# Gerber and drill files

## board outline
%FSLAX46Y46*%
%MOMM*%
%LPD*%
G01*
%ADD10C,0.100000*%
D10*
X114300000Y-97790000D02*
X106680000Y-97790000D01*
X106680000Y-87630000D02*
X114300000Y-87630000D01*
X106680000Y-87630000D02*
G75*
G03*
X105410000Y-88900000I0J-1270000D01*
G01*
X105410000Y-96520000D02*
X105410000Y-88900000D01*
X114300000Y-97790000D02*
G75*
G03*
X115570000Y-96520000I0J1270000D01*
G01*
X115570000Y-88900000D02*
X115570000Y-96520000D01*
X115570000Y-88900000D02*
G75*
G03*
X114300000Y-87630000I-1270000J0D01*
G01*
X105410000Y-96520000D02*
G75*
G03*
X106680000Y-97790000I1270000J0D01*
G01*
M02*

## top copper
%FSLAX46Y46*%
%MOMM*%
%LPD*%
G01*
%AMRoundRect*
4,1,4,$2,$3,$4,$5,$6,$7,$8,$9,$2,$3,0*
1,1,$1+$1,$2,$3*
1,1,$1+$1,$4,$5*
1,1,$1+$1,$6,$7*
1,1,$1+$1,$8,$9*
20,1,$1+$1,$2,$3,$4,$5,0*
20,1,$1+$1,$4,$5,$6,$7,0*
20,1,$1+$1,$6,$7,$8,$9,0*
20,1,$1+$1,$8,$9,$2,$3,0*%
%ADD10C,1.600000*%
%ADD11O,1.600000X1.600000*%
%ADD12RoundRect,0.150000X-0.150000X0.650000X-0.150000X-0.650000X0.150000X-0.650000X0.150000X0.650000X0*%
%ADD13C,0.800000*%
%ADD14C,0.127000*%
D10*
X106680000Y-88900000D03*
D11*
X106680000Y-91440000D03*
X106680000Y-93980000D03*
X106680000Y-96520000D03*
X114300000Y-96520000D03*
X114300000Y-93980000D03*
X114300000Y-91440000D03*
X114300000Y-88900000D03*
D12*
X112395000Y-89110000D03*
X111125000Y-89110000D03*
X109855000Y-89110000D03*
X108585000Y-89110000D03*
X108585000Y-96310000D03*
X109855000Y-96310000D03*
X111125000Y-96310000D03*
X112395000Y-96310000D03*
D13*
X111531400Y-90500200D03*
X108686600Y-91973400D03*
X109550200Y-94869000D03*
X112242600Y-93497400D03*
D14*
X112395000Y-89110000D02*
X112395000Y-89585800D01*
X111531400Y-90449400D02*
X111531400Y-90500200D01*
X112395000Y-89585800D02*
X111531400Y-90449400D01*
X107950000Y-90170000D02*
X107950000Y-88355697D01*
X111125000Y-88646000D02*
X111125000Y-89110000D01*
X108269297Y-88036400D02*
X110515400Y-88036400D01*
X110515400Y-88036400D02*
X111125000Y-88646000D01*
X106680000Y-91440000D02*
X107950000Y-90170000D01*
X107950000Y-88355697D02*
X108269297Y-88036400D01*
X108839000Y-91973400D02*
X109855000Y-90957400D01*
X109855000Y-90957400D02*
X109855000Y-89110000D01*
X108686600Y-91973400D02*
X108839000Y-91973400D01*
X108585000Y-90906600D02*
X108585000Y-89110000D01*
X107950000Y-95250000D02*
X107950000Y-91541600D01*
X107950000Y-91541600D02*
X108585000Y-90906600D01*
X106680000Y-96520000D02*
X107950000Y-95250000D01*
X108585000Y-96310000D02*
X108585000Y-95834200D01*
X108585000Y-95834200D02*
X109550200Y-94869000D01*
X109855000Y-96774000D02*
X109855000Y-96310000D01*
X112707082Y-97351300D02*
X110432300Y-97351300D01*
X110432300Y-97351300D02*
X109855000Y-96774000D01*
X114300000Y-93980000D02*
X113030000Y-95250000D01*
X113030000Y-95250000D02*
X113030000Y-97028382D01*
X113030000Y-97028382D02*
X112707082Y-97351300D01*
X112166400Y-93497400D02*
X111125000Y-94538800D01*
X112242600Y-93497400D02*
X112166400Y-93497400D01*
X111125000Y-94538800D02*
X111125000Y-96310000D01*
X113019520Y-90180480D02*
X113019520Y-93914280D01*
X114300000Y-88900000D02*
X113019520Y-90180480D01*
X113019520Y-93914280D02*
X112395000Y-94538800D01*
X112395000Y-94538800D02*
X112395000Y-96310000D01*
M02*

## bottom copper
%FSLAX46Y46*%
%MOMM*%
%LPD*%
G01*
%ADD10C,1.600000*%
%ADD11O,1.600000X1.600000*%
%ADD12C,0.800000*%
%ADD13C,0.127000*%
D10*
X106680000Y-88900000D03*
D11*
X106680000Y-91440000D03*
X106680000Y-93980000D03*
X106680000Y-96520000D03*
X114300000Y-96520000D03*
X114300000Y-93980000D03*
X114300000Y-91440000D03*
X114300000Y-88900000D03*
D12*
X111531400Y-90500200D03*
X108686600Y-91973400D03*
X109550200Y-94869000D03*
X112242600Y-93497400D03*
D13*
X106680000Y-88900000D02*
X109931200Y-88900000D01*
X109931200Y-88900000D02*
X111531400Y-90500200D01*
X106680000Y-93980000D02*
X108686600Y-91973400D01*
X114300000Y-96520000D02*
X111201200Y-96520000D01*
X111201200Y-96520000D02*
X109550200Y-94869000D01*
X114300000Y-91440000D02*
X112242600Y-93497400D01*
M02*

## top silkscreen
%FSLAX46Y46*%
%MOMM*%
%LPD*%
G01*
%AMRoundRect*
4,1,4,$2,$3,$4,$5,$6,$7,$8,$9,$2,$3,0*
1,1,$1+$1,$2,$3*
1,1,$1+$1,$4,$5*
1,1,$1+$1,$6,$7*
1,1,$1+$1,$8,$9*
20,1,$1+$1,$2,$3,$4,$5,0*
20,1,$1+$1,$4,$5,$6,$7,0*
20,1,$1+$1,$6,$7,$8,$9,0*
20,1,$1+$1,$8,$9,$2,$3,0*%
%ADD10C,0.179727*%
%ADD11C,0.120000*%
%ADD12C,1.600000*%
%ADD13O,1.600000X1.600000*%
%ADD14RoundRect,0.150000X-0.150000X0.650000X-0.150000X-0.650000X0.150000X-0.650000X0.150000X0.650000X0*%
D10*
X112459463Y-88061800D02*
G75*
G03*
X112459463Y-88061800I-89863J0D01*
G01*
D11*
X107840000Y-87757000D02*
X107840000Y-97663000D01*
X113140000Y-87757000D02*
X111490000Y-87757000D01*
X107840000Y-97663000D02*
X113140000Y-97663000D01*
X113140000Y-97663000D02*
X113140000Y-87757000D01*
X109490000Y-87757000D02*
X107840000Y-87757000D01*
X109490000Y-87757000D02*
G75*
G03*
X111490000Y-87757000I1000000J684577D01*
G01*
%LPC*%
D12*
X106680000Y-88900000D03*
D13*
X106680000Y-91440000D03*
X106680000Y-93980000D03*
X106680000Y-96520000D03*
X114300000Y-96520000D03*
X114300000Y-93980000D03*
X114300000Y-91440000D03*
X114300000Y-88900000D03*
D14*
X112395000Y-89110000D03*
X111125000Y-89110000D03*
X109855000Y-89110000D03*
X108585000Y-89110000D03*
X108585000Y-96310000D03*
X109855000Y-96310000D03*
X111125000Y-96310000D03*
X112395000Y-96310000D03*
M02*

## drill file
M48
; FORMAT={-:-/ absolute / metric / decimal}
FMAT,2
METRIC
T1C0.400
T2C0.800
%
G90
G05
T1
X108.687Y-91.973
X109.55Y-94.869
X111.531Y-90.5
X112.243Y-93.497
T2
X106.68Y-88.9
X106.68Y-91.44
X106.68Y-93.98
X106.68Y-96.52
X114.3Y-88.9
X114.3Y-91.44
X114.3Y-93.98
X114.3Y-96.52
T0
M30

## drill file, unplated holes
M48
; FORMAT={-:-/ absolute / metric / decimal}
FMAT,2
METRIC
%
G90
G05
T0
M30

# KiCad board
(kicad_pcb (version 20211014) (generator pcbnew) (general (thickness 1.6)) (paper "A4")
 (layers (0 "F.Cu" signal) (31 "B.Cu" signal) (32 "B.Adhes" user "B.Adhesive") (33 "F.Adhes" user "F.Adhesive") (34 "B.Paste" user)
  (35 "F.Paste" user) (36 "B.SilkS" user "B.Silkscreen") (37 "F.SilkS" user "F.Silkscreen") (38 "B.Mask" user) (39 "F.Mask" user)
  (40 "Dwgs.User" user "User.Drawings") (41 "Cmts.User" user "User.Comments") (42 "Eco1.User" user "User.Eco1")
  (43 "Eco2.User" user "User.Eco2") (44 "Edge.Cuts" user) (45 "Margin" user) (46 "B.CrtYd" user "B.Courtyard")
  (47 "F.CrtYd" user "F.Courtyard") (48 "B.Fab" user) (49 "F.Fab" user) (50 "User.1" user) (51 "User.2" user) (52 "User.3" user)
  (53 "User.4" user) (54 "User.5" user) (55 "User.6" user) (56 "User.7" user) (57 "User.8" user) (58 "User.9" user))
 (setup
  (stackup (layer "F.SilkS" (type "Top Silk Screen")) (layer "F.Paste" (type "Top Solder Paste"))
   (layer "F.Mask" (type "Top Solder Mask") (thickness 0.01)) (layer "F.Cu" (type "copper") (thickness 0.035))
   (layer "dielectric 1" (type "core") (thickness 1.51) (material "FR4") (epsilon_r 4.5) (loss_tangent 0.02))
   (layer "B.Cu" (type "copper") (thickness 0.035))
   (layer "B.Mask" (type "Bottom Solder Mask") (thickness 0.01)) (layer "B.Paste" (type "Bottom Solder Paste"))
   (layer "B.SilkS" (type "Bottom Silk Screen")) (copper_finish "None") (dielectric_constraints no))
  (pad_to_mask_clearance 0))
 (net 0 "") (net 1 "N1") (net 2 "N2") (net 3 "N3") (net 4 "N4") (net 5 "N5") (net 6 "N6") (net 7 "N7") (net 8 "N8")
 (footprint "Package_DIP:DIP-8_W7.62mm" (layer "F.Cu") (at 106.68 88.9)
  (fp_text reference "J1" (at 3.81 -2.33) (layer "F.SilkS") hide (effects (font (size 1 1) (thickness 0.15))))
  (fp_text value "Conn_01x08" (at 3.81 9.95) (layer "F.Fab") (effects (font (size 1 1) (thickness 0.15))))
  (fp_line (start 1.16 -1.143) (end 1.16 8.763) (layer "F.SilkS") (width 0.12))
  (fp_line (start 6.46 -1.143) (end 4.81 -1.143) (layer "F.SilkS") (width 0.12))
  (fp_line (start 1.16 8.763) (end 6.46 8.763) (layer "F.SilkS") (width 0.12))
  (fp_line (start 6.46 8.763) (end 6.46 -1.143) (layer "F.SilkS") (width 0.12))
  (fp_line (start 2.81 -1.143) (end 1.16 -1.143) (layer "F.SilkS") (width 0.12))
  (fp_arc (start 4.81 -1.143) (mid 3.81 -0.6157) (end 2.81 -1.143) (layer "F.SilkS") (width 0.12))
  (pad "1" thru_hole circle (at 0 0) (size 1.6 1.6) (drill 0.8) (layers *.Cu *.Mask) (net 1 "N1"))
  (pad "2" thru_hole oval (at 0 2.54) (size 1.6 1.6) (drill 0.8) (layers *.Cu *.Mask) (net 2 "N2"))
  (pad "3" thru_hole oval (at 0 5.08) (size 1.6 1.6) (drill 0.8) (layers *.Cu *.Mask) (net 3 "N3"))
  (pad "4" thru_hole oval (at 0 7.62) (size 1.6 1.6) (drill 0.8) (layers *.Cu *.Mask) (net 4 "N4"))
  (pad "5" thru_hole oval (at 7.62 7.62) (size 1.6 1.6) (drill 0.8) (layers *.Cu *.Mask) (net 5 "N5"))
  (pad "6" thru_hole oval (at 7.62 5.08) (size 1.6 1.6) (drill 0.8) (layers *.Cu *.Mask) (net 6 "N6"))
  (pad "7" thru_hole oval (at 7.62 2.54) (size 1.6 1.6) (drill 0.8) (layers *.Cu *.Mask) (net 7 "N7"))
  (pad "8" thru_hole oval (at 7.62 0) (size 1.6 1.6) (drill 0.8) (layers *.Cu *.Mask) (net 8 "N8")))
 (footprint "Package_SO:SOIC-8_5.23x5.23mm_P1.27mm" (layer "F.Cu") (at 110.49 92.71 -90)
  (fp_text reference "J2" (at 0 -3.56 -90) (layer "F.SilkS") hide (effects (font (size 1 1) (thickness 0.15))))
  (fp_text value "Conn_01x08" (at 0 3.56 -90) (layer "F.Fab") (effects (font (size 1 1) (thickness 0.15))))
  (pad "1" smd roundrect (at -3.6 -1.905 270) (size 1.6 0.6) (layers "F.Cu" "F.Paste" "F.Mask") (roundrect_rratio 0.25) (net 1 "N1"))
  (pad "2" smd roundrect (at -3.6 -0.635 270) (size 1.6 0.6) (layers "F.Cu" "F.Paste" "F.Mask") (roundrect_rratio 0.25) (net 2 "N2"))
  (pad "3" smd roundrect (at -3.6 0.635 270) (size 1.6 0.6) (layers "F.Cu" "F.Paste" "F.Mask") (roundrect_rratio 0.25) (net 3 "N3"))
  (pad "4" smd roundrect (at -3.6 1.905 270) (size 1.6 0.6) (layers "F.Cu" "F.Paste" "F.Mask") (roundrect_rratio 0.25) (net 4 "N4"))
  (pad "5" smd roundrect (at 3.6 1.905 270) (size 1.6 0.6) (layers "F.Cu" "F.Paste" "F.Mask") (roundrect_rratio 0.25) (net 5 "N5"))
  (pad "6" smd roundrect (at 3.6 0.635 270) (size 1.6 0.6) (layers "F.Cu" "F.Paste" "F.Mask") (roundrect_rratio 0.25) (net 6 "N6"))
  (pad "7" smd roundrect (at 3.6 -0.635 270) (size 1.6 0.6) (layers "F.Cu" "F.Paste" "F.Mask") (roundrect_rratio 0.25) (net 7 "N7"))
  (pad "8" smd roundrect (at 3.6 -1.905 270) (size 1.6 0.6) (layers "F.Cu" "F.Paste" "F.Mask") (roundrect_rratio 0.25) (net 8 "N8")))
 (gr_circle (center 112.3696 88.0618) (end 112.4712 88.0872) (layer "F.SilkS") (width 0.15) (fill solid))
 (gr_line (start 114.3 97.79) (end 106.68 97.79) (layer "Edge.Cuts") (width 0.1))
 (gr_line (start 106.68 87.63) (end 114.3 87.63) (layer "Edge.Cuts") (width 0.1))
 (gr_arc (start 105.41 88.9) (mid 105.781974 88.001974) (end 106.68 87.63) (layer "Edge.Cuts") (width 0.1))
 (gr_line (start 105.41 96.52) (end 105.41 88.9) (layer "Edge.Cuts") (width 0.1))
 (gr_arc (start 115.57 96.52) (mid 115.198026 97.418026) (end 114.3 97.79) (layer "Edge.Cuts") (width 0.1))
 (gr_line (start 115.57 88.9) (end 115.57 96.52) (layer "Edge.Cuts") (width 0.1))
 (gr_arc (start 114.3 87.63) (mid 115.198026 88.001974) (end 115.57 88.9) (layer "Edge.Cuts") (width 0.1))
 (gr_arc (start 106.68 97.79) (mid 105.781974 97.418026) (end 105.41 96.52) (layer "Edge.Cuts") (width 0.1))
 (segment (start 112.395 89.11) (end 112.395 89.5858) (width 0.127) (layer "F.Cu") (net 1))
 (segment (start 111.5314 90.4494) (end 111.5314 90.5002) (width 0.127) (layer "F.Cu") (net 1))
 (segment (start 112.395 89.5858) (end 111.5314 90.4494) (width 0.127) (layer "F.Cu") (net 1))
 (via (at 111.5314 90.5002) (size 0.8) (drill 0.4) (layers "F.Cu" "B.Cu") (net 1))
 (segment (start 106.68 88.9) (end 109.9312 88.9) (width 0.127) (layer "B.Cu") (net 1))
 (segment (start 109.9312 88.9) (end 111.5314 90.5002) (width 0.127) (layer "B.Cu") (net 1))
 (segment (start 107.95 90.17) (end 107.95 88.355697) (width 0.127) (layer "F.Cu") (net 2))
 (segment (start 111.125 88.646) (end 111.125 89.11) (width 0.127) (layer "F.Cu") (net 2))
 (segment (start 108.269297 88.0364) (end 110.5154 88.0364) (width 0.127) (layer "F.Cu") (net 2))
 (segment (start 110.5154 88.0364) (end 111.125 88.646) (width 0.127) (layer "F.Cu") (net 2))
 (segment (start 106.68 91.44) (end 107.95 90.17) (width 0.127) (layer "F.Cu") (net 2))
 (segment (start 107.95 88.355697) (end 108.269297 88.0364) (width 0.127) (layer "F.Cu") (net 2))
 (segment (start 108.839 91.9734) (end 109.855 90.9574) (width 0.127) (layer "F.Cu") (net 3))
 (segment (start 109.855 90.9574) (end 109.855 89.11) (width 0.127) (layer "F.Cu") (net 3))
 (segment (start 108.6866 91.9734) (end 108.839 91.9734) (width 0.127) (layer "F.Cu") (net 3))
 (via (at 108.6866 91.9734) (size 0.8) (drill 0.4) (layers "F.Cu" "B.Cu") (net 3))
 (segment (start 106.68 93.98) (end 108.6866 91.9734) (width 0.127) (layer "B.Cu") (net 3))
 (segment (start 108.585 90.9066) (end 108.585 89.11) (width 0.127) (layer "F.Cu") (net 4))
 (segment (start 107.95 95.25) (end 107.95 91.5416) (width 0.127) (layer "F.Cu") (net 4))
 (segment (start 107.95 91.5416) (end 108.585 90.9066) (width 0.127) (layer "F.Cu") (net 4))
 (segment (start 106.68 96.52) (end 107.95 95.25) (width 0.127) (layer "F.Cu") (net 4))
 (segment (start 108.585 96.31) (end 108.585 95.8342) (width 0.127) (layer "F.Cu") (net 5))
 (segment (start 108.585 95.8342) (end 109.5502 94.869) (width 0.127) (layer "F.Cu") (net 5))
 (via (at 109.5502 94.869) (size 0.8) (drill 0.4) (layers "F.Cu" "B.Cu") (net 5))
 (segment (start 114.3 96.52) (end 111.2012 96.52) (width 0.127) (layer "B.Cu") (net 5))
 (segment (start 111.2012 96.52) (end 109.5502 94.869) (width 0.127) (layer "B.Cu") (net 5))
 (segment (start 109.855 96.774) (end 109.855 96.31) (width 0.127) (layer "F.Cu") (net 6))
 (segment (start 112.707082 97.3513) (end 110.4323 97.3513) (width 0.127) (layer "F.Cu") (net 6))
 (segment (start 110.4323 97.3513) (end 109.855 96.774) (width 0.127) (layer "F.Cu") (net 6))
 (segment (start 114.3 93.98) (end 113.03 95.25) (width 0.127) (layer "F.Cu") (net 6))
 (segment (start 113.03 95.25) (end 113.03 97.028382) (width 0.127) (layer "F.Cu") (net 6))
 (segment (start 113.03 97.028382) (end 112.707082 97.3513) (width 0.127) (layer "F.Cu") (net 6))
 (segment (start 112.1664 93.4974) (end 111.125 94.5388) (width 0.127) (layer "F.Cu") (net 7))
 (segment (start 112.2426 93.4974) (end 112.1664 93.4974) (width 0.127) (layer "F.Cu") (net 7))
 (segment (start 111.125 94.5388) (end 111.125 96.31) (width 0.127) (layer "F.Cu") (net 7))
 (via (at 112.2426 93.4974) (size 0.8) (drill 0.4) (layers "F.Cu" "B.Cu") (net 7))
 (segment (start 114.3 91.44) (end 112.2426 93.4974) (width 0.127) (layer "B.Cu") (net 7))
 (segment (start 113.01952 90.18048) (end 113.01952 93.91428) (width 0.127) (layer "F.Cu") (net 8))
 (segment (start 114.3 88.9) (end 113.01952 90.18048) (width 0.127) (layer "F.Cu") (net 8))
 (segment (start 113.01952 93.91428) (end 112.395 94.5388) (width 0.127) (layer "F.Cu") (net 8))
 (segment (start 112.395 94.5388) (end 112.395 96.31) (width 0.127) (layer "F.Cu") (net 8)))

